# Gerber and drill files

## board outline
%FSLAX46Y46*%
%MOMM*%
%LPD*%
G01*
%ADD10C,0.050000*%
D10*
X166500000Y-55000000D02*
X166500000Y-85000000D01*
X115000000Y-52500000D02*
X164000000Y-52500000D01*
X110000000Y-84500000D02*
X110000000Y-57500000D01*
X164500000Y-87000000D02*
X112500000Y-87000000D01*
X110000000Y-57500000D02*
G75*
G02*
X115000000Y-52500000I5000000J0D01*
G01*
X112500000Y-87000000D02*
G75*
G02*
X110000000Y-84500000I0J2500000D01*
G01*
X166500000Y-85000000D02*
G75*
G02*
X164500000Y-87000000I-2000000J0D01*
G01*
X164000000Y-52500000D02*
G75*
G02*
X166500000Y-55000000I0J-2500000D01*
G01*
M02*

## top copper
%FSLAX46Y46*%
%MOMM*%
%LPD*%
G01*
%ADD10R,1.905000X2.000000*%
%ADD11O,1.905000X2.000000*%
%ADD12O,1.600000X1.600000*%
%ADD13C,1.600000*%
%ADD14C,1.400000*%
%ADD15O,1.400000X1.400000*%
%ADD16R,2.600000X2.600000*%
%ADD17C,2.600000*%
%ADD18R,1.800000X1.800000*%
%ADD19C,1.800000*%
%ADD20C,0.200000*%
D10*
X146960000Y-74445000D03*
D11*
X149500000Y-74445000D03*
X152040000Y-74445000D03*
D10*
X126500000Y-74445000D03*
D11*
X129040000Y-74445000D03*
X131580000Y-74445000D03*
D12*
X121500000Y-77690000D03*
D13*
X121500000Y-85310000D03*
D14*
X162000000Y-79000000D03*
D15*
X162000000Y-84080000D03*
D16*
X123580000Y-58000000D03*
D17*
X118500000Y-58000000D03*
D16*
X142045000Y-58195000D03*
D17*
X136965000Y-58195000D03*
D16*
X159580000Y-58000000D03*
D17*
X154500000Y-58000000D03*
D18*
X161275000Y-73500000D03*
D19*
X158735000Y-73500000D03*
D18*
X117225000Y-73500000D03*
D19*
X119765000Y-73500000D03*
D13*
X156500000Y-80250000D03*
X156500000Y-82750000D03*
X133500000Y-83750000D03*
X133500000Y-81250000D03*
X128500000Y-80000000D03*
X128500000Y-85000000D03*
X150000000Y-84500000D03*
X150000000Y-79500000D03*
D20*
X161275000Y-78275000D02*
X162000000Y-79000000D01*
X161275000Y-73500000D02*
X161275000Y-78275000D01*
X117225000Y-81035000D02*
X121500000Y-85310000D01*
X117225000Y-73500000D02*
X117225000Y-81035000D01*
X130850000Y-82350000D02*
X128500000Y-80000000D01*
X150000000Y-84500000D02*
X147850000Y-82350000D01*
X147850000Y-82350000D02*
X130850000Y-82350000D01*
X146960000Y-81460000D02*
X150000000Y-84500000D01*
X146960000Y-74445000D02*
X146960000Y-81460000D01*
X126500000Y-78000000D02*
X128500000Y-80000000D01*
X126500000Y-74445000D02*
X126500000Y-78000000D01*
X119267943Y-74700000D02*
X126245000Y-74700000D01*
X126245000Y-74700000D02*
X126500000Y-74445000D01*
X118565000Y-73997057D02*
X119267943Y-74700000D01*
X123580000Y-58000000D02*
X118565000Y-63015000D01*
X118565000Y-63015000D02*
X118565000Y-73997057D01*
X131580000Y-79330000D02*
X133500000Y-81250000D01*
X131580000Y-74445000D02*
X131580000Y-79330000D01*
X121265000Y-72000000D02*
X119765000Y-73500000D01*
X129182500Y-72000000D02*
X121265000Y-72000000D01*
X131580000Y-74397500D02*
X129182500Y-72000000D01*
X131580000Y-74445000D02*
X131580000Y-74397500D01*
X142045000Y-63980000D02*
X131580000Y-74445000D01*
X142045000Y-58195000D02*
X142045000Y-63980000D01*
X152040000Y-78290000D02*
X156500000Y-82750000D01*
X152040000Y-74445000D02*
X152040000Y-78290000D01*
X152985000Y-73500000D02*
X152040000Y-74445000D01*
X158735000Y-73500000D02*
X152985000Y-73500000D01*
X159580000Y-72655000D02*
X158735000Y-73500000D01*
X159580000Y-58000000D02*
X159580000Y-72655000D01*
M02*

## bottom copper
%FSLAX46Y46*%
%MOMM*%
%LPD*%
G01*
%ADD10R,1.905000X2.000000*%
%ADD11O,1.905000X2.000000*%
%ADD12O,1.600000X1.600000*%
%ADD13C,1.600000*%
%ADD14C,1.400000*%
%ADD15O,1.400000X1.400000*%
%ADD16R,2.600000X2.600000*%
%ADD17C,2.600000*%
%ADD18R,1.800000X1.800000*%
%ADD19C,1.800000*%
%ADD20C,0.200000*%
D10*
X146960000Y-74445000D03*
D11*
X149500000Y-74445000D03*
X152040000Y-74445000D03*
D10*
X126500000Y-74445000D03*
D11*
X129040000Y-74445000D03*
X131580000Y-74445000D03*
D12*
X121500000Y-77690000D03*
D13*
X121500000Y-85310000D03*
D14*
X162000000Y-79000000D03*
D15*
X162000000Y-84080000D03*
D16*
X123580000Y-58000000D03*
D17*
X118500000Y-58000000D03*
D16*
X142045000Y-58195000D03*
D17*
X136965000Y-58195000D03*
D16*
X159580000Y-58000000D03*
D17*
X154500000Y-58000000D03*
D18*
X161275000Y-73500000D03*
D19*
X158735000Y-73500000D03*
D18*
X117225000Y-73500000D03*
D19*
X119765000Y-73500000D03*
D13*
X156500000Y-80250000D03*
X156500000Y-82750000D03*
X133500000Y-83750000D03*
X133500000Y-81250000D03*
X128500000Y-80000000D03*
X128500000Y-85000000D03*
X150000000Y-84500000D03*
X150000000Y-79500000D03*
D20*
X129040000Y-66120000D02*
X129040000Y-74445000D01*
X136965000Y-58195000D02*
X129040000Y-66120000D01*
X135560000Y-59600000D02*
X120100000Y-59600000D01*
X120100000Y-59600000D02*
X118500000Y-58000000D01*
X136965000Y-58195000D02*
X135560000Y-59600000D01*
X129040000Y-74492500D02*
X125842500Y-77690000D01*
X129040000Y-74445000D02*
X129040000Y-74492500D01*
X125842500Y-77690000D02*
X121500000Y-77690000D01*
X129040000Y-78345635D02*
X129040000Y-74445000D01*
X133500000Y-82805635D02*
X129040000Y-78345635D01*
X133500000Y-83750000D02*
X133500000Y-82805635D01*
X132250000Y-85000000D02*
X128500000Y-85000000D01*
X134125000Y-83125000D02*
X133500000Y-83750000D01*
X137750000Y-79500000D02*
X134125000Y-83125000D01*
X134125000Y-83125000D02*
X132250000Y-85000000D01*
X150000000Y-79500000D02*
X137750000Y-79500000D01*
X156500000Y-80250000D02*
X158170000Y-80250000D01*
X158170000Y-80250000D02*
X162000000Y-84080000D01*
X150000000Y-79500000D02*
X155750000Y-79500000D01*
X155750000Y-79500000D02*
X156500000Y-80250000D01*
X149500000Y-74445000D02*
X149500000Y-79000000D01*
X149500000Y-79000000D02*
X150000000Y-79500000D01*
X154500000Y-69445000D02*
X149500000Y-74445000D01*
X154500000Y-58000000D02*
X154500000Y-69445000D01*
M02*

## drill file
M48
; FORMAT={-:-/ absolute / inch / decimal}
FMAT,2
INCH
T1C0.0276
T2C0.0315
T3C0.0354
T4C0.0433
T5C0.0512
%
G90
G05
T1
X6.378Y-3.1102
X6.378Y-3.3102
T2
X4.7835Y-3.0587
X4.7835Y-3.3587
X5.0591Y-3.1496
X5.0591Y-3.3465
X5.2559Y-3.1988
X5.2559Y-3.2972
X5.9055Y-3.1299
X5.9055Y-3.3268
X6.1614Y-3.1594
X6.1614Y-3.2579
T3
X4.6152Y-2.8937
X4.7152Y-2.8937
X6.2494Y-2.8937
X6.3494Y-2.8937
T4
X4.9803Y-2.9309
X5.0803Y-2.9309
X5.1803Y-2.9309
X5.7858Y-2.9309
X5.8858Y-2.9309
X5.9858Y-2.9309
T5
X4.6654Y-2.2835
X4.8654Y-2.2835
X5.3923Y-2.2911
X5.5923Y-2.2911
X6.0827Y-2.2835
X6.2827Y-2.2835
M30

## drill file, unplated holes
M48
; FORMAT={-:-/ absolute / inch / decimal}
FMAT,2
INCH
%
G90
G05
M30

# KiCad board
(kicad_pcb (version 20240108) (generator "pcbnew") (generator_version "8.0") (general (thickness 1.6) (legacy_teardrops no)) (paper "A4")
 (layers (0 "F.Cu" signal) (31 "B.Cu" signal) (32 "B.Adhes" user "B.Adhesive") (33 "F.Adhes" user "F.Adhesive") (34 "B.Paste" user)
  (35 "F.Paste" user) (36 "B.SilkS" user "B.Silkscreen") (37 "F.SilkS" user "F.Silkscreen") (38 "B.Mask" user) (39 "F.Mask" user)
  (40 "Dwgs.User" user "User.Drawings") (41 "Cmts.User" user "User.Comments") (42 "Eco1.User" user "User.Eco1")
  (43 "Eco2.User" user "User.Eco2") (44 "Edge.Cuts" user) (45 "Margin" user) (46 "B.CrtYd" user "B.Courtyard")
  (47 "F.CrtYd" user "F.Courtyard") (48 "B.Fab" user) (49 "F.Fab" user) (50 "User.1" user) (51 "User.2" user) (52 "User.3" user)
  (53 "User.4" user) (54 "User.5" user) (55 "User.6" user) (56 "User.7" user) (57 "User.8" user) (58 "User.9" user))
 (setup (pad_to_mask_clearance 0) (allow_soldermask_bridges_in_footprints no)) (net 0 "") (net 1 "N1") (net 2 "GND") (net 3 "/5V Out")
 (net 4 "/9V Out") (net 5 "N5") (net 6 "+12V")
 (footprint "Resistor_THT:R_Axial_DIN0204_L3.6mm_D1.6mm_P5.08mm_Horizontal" (layer "F.Cu") (at 162 79 -90)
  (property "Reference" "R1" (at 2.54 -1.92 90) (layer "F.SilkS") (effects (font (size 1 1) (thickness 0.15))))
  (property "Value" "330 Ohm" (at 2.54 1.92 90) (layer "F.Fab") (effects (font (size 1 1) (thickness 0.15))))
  (pad "1" thru_hole circle (at 0 0 270) (size 1.4 1.4) (drill 0.7) (layers "*.Cu" "*.Mask") (remove_unused_layers no) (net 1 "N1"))
  (pad "2" thru_hole oval (at 5.08 0 270) (size 1.4 1.4) (drill 0.7) (layers "*.Cu" "*.Mask") (remove_unused_layers no) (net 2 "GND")))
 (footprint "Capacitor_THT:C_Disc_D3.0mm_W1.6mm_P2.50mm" (layer "F.Cu") (at 156.5 82.75 90)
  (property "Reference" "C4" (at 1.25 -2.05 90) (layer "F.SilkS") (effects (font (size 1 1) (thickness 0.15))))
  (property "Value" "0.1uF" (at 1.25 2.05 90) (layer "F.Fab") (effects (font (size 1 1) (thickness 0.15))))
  (pad "1" thru_hole circle (at 0 0 90) (size 1.6 1.6) (drill 0.8) (layers "*.Cu" "*.Mask") (remove_unused_layers no) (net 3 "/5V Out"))
  (pad "2" thru_hole circle (at 2.5 0 90) (size 1.6 1.6) (drill 0.8) (layers "*.Cu" "*.Mask") (remove_unused_layers no) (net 2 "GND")))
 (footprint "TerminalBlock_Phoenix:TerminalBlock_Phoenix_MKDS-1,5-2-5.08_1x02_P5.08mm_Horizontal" (layer "F.Cu") (at 142.045 58.195 180)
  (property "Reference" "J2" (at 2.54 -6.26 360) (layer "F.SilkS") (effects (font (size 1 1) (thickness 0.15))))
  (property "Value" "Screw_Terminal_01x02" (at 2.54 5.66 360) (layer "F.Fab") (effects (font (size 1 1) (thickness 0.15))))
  (pad "1" thru_hole rect (at 0 0 180) (size 2.6 2.6) (drill 1.3) (layers "*.Cu" "*.Mask") (remove_unused_layers no) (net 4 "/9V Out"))
  (pad "2" thru_hole circle (at 5.08 0 180) (size 2.6 2.6) (drill 1.3) (layers "*.Cu" "*.Mask") (remove_unused_layers no) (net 2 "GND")))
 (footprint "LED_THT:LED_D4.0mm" (layer "F.Cu") (at 117.225 73.5)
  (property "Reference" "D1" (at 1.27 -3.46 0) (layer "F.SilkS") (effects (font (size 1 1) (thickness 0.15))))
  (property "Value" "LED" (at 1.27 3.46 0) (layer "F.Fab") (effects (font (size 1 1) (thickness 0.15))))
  (pad "1" thru_hole rect (at 0 0) (size 1.8 1.8) (drill 0.9) (layers "*.Cu" "*.Mask") (remove_unused_layers no) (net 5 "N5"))
  (pad "2" thru_hole circle (at 2.54 0) (size 1.8 1.8) (drill 0.9) (layers "*.Cu" "*.Mask") (remove_unused_layers no) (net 4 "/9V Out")))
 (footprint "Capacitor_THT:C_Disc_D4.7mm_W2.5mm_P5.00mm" (layer "F.Cu") (at 128.5 80 -90)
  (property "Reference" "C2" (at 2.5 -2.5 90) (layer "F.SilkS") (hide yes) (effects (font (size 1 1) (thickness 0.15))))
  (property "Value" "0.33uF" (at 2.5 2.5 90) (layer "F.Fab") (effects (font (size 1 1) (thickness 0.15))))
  (pad "1" thru_hole circle (at 0 0 270) (size 1.6 1.6) (drill 0.8) (layers "*.Cu" "*.Mask") (remove_unused_layers no) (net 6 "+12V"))
  (pad "2" thru_hole circle (at 5 0 270) (size 1.6 1.6) (drill 0.8) (layers "*.Cu" "*.Mask") (remove_unused_layers no) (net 2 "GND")))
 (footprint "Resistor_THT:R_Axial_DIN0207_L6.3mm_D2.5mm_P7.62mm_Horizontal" (layer "F.Cu") (at 121.5 85.31 90)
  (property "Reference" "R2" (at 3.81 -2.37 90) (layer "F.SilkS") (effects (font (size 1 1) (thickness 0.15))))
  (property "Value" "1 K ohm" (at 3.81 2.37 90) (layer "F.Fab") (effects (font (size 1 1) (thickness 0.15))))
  (pad "1" thru_hole circle (at 0 0 90) (size 1.6 1.6) (drill 0.8) (layers "*.Cu" "*.Mask") (remove_unused_layers no) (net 5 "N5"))
  (pad "2" thru_hole oval (at 7.62 0 90) (size 1.6 1.6) (drill 0.8) (layers "*.Cu" "*.Mask") (remove_unused_layers no) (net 2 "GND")))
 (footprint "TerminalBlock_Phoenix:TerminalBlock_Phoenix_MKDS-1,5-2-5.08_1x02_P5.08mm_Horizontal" (layer "F.Cu") (at 123.58 58 180)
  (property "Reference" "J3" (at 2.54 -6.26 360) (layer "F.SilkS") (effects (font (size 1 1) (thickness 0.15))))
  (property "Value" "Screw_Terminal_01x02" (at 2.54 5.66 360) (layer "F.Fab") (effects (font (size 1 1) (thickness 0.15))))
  (pad "1" thru_hole rect (at 0 0 180) (size 2.6 2.6) (drill 1.3) (layers "*.Cu" "*.Mask") (remove_unused_layers no) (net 6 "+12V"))
  (pad "2" thru_hole circle (at 5.08 0 180) (size 2.6 2.6) (drill 1.3) (layers "*.Cu" "*.Mask") (remove_unused_layers no) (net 2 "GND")))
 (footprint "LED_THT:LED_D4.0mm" (layer "F.Cu") (at 161.275 73.5 180)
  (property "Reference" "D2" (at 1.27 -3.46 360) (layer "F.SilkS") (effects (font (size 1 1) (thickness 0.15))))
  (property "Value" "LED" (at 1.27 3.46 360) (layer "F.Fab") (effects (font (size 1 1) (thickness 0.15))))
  (pad "1" thru_hole rect (at 0 0 180) (size 1.8 1.8) (drill 0.9) (layers "*.Cu" "*.Mask") (remove_unused_layers no) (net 1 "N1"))
  (pad "2" thru_hole circle (at 2.54 0 180) (size 1.8 1.8) (drill 0.9) (layers "*.Cu" "*.Mask") (remove_unused_layers no) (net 3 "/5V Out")))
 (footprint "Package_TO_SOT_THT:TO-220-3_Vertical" (layer "F.Cu") (at 126.5 74.445)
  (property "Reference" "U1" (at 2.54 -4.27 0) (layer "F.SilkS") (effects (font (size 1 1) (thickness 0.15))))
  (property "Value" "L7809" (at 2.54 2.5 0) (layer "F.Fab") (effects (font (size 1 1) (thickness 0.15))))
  (pad "1" thru_hole rect (at 0 0) (size 1.905 2) (drill 1.1) (layers "*.Cu" "*.Mask") (remove_unused_layers no) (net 6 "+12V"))
  (pad "2" thru_hole oval (at 2.54 0) (size 1.905 2) (drill 1.1) (layers "*.Cu" "*.Mask") (remove_unused_layers no) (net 2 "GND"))
  (pad "3" thru_hole oval (at 5.08 0) (size 1.905 2) (drill 1.1) (layers "*.Cu" "*.Mask") (remove_unused_layers no) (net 4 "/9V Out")))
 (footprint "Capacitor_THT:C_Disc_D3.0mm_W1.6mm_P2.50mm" (layer "F.Cu") (at 133.5 81.25 -90)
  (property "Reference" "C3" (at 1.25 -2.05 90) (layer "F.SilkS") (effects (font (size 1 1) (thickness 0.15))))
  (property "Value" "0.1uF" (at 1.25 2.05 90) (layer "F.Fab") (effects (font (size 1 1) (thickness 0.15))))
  (pad "1" thru_hole circle (at 0 0 270) (size 1.6 1.6) (drill 0.8) (layers "*.Cu" "*.Mask") (remove_unused_layers no) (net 4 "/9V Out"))
  (pad "2" thru_hole circle (at 2.5 0 270) (size 1.6 1.6) (drill 0.8) (layers "*.Cu" "*.Mask") (remove_unused_layers no) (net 2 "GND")))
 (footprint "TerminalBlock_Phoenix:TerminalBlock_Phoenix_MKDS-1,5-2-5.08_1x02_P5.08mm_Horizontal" (layer "F.Cu") (at 159.58 58 180)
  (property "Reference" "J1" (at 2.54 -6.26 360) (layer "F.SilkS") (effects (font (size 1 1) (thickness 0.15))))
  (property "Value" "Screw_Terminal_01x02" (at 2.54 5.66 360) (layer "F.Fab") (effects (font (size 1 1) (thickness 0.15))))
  (pad "1" thru_hole rect (at 0 0 180) (size 2.6 2.6) (drill 1.3) (layers "*.Cu" "*.Mask") (remove_unused_layers no) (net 3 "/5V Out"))
  (pad "2" thru_hole circle (at 5.08 0 180) (size 2.6 2.6) (drill 1.3) (layers "*.Cu" "*.Mask") (remove_unused_layers no) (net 2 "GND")))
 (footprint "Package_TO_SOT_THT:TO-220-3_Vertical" (layer "F.Cu") (at 146.96 74.445)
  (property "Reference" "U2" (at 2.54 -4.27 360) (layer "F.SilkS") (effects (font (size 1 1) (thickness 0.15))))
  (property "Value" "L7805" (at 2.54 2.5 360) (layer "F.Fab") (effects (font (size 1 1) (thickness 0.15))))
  (pad "1" thru_hole rect (at 0 0) (size 1.905 2) (drill 1.1) (layers "*.Cu" "*.Mask") (remove_unused_layers no) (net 6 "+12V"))
  (pad "2" thru_hole oval (at 2.54 0) (size 1.905 2) (drill 1.1) (layers "*.Cu" "*.Mask") (remove_unused_layers no) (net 2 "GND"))
  (pad "3" thru_hole oval (at 5.08 0) (size 1.905 2) (drill 1.1) (layers "*.Cu" "*.Mask") (remove_unused_layers no) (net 3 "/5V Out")))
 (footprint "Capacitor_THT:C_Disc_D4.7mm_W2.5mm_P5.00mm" (layer "F.Cu") (at 150 84.5 90)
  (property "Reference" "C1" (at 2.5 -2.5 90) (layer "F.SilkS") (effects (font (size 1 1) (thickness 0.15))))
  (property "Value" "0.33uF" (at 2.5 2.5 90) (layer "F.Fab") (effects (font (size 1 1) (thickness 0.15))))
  (pad "1" thru_hole circle (at 0 0 90) (size 1.6 1.6) (drill 0.8) (layers "*.Cu" "*.Mask") (remove_unused_layers no) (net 6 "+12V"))
  (pad "2" thru_hole circle (at 5 0 90) (size 1.6 1.6) (drill 0.8) (layers "*.Cu" "*.Mask") (remove_unused_layers no) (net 2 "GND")))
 (gr_arc (start 110 57.5) (mid 111.464466 53.964466) (end 115 52.5) (stroke (width 0.05) (type default)) (layer "Edge.Cuts"))
 (gr_arc (start 112.5 87) (mid 110.732233 86.267767) (end 110 84.5) (stroke (width 0.05) (type default)) (layer "Edge.Cuts"))
 (gr_line (start 115 52.5) (end 164 52.5) (stroke (width 0.05) (type default)) (layer "Edge.Cuts"))
 (gr_line (start 110 84.5) (end 110 57.5) (stroke (width 0.05) (type default)) (layer "Edge.Cuts"))
 (gr_line (start 166.5 55) (end 166.5 85) (stroke (width 0.05) (type default)) (layer "Edge.Cuts"))
 (gr_line (start 164.5 87) (end 112.5 87) (stroke (width 0.05) (type default)) (layer "Edge.Cuts"))
 (gr_arc (start 164 52.5) (mid 165.767767 53.232233) (end 166.5 55) (stroke (width 0.05) (type default)) (layer "Edge.Cuts"))
 (gr_arc (start 166.5 85) (mid 165.914214 86.414214) (end 164.5 87) (stroke (width 0.05) (type default)) (layer "Edge.Cuts"))
 (segment (start 123.58 58) (end 118.565 63.015) (width 0.2) (layer "F.Cu") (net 6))
 (segment (start 150 84.5) (end 147.85 82.35) (width 0.2) (layer "F.Cu") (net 6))
 (segment (start 119.267943 74.7) (end 126.245 74.7) (width 0.2) (layer "F.Cu") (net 6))
 (segment (start 130.85 82.35) (end 128.5 80) (width 0.2) (layer "F.Cu") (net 6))
 (segment (start 147.85 82.35) (end 130.85 82.35) (width 0.2) (layer "F.Cu") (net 6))
 (segment (start 126.5 78) (end 128.5 80) (width 0.2) (layer "F.Cu") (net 6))
 (segment (start 126.5 74.445) (end 126.5 78) (width 0.2) (layer "F.Cu") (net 6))
 (segment (start 146.96 74.445) (end 146.96 81.46) (width 0.2) (layer "F.Cu") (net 6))
 (segment (start 118.565 63.015) (end 118.565 73.997057) (width 0.2) (layer "F.Cu") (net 6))
 (segment (start 118.565 73.997057) (end 119.267943 74.7) (width 0.2) (layer "F.Cu") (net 6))
 (segment (start 146.96 81.46) (end 150 84.5) (width 0.2) (layer "F.Cu") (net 6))
 (segment (start 126.245 74.7) (end 126.5 74.445) (width 0.2) (layer "F.Cu") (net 6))
 (segment (start 132.25 85) (end 128.5 85) (width 0.2) (layer "B.Cu") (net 2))
 (segment (start 150 79.5) (end 137.75 79.5) (width 0.2) (layer "B.Cu") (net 2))
 (segment (start 125.8425 77.69) (end 121.5 77.69) (width 0.2) (layer "B.Cu") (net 2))
 (segment (start 134.125 83.125) (end 133.5 83.75) (width 0.2) (layer "B.Cu") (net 2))
 (segment (start 129.04 74.4925) (end 125.8425 77.69) (width 0.2) (layer "B.Cu") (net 2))
 (segment (start 120.1 59.6) (end 118.5 58) (width 0.2) (layer "B.Cu") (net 2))
 (segment (start 133.5 83.75) (end 133.5 82.805635) (width 0.2) (layer "B.Cu") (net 2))
 (segment (start 135.56 59.6) (end 120.1 59.6) (width 0.2) (layer "B.Cu") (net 2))
 (segment (start 155.75 79.5) (end 156.5 80.25) (width 0.2) (layer "B.Cu") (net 2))
 (segment (start 129.04 66.12) (end 129.04 74.445) (width 0.2) (layer "B.Cu") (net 2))
 (segment (start 154.5 69.445) (end 149.5 74.445) (width 0.2) (layer "B.Cu") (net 2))
 (segment (start 158.17 80.25) (end 162 84.08) (width 0.2) (layer "B.Cu") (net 2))
 (segment (start 154.5 58) (end 154.5 69.445) (width 0.2) (layer "B.Cu") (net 2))
 (segment (start 129.04 74.445) (end 129.04 74.4925) (width 0.2) (layer "B.Cu") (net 2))
 (segment (start 149.5 74.445) (end 149.5 79) (width 0.2) (layer "B.Cu") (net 2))
 (segment (start 133.5 82.805635) (end 129.04 78.345635) (width 0.2) (layer "B.Cu") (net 2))
 (segment (start 150 79.5) (end 155.75 79.5) (width 0.2) (layer "B.Cu") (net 2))
 (segment (start 129.04 78.345635) (end 129.04 74.445) (width 0.2) (layer "B.Cu") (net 2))
 (segment (start 149.5 79) (end 150 79.5) (width 0.2) (layer "B.Cu") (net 2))
 (segment (start 134.125 83.125) (end 132.25 85) (width 0.2) (layer "B.Cu") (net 2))
 (segment (start 136.965 58.195) (end 129.04 66.12) (width 0.2) (layer "B.Cu") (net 2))
 (segment (start 136.965 58.195) (end 135.56 59.6) (width 0.2) (layer "B.Cu") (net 2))
 (segment (start 137.75 79.5) (end 134.125 83.125) (width 0.2) (layer "B.Cu") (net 2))
 (segment (start 156.5 80.25) (end 158.17 80.25) (width 0.2) (layer "B.Cu") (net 2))
 (segment (start 131.58 74.445) (end 131.58 79.33) (width 0.2) (layer "F.Cu") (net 4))
 (segment (start 142.045 63.98) (end 131.58 74.445) (width 0.2) (layer "F.Cu") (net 4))
 (segment (start 131.58 74.445) (end 131.58 74.3975) (width 0.2) (layer "F.Cu") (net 4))
 (segment (start 129.1825 72) (end 121.265 72) (width 0.2) (layer "F.Cu") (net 4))
 (segment (start 142.045 58.195) (end 142.045 63.98) (width 0.2) (layer "F.Cu") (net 4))
 (segment (start 131.58 74.3975) (end 129.1825 72) (width 0.2) (layer "F.Cu") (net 4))
 (segment (start 121.265 72) (end 119.765 73.5) (width 0.2) (layer "F.Cu") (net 4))
 (segment (start 131.58 79.33) (end 133.5 81.25) (width 0.2) (layer "F.Cu") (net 4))
 (segment (start 152.04 78.29) (end 156.5 82.75) (width 0.2) (layer "F.Cu") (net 3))
 (segment (start 152.985 73.5) (end 152.04 74.445) (width 0.2) (layer "F.Cu") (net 3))
 (segment (start 159.58 72.655) (end 158.735 73.5) (width 0.2) (layer "F.Cu") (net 3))
 (segment (start 159.58 58) (end 159.58 72.655) (width 0.2) (layer "F.Cu") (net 3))
 (segment (start 152.04 74.445) (end 152.04 78.29) (width 0.2) (layer "F.Cu") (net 3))
 (segment (start 158.735 73.5) (end 152.985 73.5) (width 0.2) (layer "F.Cu") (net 3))
 (segment (start 117.225 73.5) (end 117.225 81.035) (width 0.2) (layer "F.Cu") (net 5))
 (segment (start 117.225 81.035) (end 121.5 85.31) (width 0.2) (layer "F.Cu") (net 5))
 (segment (start 161.275 78.275) (end 162 79) (width 0.2) (layer "F.Cu") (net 1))
 (segment (start 161.275 73.5) (end 161.275 78.275) (width 0.2) (layer "F.Cu") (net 1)))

